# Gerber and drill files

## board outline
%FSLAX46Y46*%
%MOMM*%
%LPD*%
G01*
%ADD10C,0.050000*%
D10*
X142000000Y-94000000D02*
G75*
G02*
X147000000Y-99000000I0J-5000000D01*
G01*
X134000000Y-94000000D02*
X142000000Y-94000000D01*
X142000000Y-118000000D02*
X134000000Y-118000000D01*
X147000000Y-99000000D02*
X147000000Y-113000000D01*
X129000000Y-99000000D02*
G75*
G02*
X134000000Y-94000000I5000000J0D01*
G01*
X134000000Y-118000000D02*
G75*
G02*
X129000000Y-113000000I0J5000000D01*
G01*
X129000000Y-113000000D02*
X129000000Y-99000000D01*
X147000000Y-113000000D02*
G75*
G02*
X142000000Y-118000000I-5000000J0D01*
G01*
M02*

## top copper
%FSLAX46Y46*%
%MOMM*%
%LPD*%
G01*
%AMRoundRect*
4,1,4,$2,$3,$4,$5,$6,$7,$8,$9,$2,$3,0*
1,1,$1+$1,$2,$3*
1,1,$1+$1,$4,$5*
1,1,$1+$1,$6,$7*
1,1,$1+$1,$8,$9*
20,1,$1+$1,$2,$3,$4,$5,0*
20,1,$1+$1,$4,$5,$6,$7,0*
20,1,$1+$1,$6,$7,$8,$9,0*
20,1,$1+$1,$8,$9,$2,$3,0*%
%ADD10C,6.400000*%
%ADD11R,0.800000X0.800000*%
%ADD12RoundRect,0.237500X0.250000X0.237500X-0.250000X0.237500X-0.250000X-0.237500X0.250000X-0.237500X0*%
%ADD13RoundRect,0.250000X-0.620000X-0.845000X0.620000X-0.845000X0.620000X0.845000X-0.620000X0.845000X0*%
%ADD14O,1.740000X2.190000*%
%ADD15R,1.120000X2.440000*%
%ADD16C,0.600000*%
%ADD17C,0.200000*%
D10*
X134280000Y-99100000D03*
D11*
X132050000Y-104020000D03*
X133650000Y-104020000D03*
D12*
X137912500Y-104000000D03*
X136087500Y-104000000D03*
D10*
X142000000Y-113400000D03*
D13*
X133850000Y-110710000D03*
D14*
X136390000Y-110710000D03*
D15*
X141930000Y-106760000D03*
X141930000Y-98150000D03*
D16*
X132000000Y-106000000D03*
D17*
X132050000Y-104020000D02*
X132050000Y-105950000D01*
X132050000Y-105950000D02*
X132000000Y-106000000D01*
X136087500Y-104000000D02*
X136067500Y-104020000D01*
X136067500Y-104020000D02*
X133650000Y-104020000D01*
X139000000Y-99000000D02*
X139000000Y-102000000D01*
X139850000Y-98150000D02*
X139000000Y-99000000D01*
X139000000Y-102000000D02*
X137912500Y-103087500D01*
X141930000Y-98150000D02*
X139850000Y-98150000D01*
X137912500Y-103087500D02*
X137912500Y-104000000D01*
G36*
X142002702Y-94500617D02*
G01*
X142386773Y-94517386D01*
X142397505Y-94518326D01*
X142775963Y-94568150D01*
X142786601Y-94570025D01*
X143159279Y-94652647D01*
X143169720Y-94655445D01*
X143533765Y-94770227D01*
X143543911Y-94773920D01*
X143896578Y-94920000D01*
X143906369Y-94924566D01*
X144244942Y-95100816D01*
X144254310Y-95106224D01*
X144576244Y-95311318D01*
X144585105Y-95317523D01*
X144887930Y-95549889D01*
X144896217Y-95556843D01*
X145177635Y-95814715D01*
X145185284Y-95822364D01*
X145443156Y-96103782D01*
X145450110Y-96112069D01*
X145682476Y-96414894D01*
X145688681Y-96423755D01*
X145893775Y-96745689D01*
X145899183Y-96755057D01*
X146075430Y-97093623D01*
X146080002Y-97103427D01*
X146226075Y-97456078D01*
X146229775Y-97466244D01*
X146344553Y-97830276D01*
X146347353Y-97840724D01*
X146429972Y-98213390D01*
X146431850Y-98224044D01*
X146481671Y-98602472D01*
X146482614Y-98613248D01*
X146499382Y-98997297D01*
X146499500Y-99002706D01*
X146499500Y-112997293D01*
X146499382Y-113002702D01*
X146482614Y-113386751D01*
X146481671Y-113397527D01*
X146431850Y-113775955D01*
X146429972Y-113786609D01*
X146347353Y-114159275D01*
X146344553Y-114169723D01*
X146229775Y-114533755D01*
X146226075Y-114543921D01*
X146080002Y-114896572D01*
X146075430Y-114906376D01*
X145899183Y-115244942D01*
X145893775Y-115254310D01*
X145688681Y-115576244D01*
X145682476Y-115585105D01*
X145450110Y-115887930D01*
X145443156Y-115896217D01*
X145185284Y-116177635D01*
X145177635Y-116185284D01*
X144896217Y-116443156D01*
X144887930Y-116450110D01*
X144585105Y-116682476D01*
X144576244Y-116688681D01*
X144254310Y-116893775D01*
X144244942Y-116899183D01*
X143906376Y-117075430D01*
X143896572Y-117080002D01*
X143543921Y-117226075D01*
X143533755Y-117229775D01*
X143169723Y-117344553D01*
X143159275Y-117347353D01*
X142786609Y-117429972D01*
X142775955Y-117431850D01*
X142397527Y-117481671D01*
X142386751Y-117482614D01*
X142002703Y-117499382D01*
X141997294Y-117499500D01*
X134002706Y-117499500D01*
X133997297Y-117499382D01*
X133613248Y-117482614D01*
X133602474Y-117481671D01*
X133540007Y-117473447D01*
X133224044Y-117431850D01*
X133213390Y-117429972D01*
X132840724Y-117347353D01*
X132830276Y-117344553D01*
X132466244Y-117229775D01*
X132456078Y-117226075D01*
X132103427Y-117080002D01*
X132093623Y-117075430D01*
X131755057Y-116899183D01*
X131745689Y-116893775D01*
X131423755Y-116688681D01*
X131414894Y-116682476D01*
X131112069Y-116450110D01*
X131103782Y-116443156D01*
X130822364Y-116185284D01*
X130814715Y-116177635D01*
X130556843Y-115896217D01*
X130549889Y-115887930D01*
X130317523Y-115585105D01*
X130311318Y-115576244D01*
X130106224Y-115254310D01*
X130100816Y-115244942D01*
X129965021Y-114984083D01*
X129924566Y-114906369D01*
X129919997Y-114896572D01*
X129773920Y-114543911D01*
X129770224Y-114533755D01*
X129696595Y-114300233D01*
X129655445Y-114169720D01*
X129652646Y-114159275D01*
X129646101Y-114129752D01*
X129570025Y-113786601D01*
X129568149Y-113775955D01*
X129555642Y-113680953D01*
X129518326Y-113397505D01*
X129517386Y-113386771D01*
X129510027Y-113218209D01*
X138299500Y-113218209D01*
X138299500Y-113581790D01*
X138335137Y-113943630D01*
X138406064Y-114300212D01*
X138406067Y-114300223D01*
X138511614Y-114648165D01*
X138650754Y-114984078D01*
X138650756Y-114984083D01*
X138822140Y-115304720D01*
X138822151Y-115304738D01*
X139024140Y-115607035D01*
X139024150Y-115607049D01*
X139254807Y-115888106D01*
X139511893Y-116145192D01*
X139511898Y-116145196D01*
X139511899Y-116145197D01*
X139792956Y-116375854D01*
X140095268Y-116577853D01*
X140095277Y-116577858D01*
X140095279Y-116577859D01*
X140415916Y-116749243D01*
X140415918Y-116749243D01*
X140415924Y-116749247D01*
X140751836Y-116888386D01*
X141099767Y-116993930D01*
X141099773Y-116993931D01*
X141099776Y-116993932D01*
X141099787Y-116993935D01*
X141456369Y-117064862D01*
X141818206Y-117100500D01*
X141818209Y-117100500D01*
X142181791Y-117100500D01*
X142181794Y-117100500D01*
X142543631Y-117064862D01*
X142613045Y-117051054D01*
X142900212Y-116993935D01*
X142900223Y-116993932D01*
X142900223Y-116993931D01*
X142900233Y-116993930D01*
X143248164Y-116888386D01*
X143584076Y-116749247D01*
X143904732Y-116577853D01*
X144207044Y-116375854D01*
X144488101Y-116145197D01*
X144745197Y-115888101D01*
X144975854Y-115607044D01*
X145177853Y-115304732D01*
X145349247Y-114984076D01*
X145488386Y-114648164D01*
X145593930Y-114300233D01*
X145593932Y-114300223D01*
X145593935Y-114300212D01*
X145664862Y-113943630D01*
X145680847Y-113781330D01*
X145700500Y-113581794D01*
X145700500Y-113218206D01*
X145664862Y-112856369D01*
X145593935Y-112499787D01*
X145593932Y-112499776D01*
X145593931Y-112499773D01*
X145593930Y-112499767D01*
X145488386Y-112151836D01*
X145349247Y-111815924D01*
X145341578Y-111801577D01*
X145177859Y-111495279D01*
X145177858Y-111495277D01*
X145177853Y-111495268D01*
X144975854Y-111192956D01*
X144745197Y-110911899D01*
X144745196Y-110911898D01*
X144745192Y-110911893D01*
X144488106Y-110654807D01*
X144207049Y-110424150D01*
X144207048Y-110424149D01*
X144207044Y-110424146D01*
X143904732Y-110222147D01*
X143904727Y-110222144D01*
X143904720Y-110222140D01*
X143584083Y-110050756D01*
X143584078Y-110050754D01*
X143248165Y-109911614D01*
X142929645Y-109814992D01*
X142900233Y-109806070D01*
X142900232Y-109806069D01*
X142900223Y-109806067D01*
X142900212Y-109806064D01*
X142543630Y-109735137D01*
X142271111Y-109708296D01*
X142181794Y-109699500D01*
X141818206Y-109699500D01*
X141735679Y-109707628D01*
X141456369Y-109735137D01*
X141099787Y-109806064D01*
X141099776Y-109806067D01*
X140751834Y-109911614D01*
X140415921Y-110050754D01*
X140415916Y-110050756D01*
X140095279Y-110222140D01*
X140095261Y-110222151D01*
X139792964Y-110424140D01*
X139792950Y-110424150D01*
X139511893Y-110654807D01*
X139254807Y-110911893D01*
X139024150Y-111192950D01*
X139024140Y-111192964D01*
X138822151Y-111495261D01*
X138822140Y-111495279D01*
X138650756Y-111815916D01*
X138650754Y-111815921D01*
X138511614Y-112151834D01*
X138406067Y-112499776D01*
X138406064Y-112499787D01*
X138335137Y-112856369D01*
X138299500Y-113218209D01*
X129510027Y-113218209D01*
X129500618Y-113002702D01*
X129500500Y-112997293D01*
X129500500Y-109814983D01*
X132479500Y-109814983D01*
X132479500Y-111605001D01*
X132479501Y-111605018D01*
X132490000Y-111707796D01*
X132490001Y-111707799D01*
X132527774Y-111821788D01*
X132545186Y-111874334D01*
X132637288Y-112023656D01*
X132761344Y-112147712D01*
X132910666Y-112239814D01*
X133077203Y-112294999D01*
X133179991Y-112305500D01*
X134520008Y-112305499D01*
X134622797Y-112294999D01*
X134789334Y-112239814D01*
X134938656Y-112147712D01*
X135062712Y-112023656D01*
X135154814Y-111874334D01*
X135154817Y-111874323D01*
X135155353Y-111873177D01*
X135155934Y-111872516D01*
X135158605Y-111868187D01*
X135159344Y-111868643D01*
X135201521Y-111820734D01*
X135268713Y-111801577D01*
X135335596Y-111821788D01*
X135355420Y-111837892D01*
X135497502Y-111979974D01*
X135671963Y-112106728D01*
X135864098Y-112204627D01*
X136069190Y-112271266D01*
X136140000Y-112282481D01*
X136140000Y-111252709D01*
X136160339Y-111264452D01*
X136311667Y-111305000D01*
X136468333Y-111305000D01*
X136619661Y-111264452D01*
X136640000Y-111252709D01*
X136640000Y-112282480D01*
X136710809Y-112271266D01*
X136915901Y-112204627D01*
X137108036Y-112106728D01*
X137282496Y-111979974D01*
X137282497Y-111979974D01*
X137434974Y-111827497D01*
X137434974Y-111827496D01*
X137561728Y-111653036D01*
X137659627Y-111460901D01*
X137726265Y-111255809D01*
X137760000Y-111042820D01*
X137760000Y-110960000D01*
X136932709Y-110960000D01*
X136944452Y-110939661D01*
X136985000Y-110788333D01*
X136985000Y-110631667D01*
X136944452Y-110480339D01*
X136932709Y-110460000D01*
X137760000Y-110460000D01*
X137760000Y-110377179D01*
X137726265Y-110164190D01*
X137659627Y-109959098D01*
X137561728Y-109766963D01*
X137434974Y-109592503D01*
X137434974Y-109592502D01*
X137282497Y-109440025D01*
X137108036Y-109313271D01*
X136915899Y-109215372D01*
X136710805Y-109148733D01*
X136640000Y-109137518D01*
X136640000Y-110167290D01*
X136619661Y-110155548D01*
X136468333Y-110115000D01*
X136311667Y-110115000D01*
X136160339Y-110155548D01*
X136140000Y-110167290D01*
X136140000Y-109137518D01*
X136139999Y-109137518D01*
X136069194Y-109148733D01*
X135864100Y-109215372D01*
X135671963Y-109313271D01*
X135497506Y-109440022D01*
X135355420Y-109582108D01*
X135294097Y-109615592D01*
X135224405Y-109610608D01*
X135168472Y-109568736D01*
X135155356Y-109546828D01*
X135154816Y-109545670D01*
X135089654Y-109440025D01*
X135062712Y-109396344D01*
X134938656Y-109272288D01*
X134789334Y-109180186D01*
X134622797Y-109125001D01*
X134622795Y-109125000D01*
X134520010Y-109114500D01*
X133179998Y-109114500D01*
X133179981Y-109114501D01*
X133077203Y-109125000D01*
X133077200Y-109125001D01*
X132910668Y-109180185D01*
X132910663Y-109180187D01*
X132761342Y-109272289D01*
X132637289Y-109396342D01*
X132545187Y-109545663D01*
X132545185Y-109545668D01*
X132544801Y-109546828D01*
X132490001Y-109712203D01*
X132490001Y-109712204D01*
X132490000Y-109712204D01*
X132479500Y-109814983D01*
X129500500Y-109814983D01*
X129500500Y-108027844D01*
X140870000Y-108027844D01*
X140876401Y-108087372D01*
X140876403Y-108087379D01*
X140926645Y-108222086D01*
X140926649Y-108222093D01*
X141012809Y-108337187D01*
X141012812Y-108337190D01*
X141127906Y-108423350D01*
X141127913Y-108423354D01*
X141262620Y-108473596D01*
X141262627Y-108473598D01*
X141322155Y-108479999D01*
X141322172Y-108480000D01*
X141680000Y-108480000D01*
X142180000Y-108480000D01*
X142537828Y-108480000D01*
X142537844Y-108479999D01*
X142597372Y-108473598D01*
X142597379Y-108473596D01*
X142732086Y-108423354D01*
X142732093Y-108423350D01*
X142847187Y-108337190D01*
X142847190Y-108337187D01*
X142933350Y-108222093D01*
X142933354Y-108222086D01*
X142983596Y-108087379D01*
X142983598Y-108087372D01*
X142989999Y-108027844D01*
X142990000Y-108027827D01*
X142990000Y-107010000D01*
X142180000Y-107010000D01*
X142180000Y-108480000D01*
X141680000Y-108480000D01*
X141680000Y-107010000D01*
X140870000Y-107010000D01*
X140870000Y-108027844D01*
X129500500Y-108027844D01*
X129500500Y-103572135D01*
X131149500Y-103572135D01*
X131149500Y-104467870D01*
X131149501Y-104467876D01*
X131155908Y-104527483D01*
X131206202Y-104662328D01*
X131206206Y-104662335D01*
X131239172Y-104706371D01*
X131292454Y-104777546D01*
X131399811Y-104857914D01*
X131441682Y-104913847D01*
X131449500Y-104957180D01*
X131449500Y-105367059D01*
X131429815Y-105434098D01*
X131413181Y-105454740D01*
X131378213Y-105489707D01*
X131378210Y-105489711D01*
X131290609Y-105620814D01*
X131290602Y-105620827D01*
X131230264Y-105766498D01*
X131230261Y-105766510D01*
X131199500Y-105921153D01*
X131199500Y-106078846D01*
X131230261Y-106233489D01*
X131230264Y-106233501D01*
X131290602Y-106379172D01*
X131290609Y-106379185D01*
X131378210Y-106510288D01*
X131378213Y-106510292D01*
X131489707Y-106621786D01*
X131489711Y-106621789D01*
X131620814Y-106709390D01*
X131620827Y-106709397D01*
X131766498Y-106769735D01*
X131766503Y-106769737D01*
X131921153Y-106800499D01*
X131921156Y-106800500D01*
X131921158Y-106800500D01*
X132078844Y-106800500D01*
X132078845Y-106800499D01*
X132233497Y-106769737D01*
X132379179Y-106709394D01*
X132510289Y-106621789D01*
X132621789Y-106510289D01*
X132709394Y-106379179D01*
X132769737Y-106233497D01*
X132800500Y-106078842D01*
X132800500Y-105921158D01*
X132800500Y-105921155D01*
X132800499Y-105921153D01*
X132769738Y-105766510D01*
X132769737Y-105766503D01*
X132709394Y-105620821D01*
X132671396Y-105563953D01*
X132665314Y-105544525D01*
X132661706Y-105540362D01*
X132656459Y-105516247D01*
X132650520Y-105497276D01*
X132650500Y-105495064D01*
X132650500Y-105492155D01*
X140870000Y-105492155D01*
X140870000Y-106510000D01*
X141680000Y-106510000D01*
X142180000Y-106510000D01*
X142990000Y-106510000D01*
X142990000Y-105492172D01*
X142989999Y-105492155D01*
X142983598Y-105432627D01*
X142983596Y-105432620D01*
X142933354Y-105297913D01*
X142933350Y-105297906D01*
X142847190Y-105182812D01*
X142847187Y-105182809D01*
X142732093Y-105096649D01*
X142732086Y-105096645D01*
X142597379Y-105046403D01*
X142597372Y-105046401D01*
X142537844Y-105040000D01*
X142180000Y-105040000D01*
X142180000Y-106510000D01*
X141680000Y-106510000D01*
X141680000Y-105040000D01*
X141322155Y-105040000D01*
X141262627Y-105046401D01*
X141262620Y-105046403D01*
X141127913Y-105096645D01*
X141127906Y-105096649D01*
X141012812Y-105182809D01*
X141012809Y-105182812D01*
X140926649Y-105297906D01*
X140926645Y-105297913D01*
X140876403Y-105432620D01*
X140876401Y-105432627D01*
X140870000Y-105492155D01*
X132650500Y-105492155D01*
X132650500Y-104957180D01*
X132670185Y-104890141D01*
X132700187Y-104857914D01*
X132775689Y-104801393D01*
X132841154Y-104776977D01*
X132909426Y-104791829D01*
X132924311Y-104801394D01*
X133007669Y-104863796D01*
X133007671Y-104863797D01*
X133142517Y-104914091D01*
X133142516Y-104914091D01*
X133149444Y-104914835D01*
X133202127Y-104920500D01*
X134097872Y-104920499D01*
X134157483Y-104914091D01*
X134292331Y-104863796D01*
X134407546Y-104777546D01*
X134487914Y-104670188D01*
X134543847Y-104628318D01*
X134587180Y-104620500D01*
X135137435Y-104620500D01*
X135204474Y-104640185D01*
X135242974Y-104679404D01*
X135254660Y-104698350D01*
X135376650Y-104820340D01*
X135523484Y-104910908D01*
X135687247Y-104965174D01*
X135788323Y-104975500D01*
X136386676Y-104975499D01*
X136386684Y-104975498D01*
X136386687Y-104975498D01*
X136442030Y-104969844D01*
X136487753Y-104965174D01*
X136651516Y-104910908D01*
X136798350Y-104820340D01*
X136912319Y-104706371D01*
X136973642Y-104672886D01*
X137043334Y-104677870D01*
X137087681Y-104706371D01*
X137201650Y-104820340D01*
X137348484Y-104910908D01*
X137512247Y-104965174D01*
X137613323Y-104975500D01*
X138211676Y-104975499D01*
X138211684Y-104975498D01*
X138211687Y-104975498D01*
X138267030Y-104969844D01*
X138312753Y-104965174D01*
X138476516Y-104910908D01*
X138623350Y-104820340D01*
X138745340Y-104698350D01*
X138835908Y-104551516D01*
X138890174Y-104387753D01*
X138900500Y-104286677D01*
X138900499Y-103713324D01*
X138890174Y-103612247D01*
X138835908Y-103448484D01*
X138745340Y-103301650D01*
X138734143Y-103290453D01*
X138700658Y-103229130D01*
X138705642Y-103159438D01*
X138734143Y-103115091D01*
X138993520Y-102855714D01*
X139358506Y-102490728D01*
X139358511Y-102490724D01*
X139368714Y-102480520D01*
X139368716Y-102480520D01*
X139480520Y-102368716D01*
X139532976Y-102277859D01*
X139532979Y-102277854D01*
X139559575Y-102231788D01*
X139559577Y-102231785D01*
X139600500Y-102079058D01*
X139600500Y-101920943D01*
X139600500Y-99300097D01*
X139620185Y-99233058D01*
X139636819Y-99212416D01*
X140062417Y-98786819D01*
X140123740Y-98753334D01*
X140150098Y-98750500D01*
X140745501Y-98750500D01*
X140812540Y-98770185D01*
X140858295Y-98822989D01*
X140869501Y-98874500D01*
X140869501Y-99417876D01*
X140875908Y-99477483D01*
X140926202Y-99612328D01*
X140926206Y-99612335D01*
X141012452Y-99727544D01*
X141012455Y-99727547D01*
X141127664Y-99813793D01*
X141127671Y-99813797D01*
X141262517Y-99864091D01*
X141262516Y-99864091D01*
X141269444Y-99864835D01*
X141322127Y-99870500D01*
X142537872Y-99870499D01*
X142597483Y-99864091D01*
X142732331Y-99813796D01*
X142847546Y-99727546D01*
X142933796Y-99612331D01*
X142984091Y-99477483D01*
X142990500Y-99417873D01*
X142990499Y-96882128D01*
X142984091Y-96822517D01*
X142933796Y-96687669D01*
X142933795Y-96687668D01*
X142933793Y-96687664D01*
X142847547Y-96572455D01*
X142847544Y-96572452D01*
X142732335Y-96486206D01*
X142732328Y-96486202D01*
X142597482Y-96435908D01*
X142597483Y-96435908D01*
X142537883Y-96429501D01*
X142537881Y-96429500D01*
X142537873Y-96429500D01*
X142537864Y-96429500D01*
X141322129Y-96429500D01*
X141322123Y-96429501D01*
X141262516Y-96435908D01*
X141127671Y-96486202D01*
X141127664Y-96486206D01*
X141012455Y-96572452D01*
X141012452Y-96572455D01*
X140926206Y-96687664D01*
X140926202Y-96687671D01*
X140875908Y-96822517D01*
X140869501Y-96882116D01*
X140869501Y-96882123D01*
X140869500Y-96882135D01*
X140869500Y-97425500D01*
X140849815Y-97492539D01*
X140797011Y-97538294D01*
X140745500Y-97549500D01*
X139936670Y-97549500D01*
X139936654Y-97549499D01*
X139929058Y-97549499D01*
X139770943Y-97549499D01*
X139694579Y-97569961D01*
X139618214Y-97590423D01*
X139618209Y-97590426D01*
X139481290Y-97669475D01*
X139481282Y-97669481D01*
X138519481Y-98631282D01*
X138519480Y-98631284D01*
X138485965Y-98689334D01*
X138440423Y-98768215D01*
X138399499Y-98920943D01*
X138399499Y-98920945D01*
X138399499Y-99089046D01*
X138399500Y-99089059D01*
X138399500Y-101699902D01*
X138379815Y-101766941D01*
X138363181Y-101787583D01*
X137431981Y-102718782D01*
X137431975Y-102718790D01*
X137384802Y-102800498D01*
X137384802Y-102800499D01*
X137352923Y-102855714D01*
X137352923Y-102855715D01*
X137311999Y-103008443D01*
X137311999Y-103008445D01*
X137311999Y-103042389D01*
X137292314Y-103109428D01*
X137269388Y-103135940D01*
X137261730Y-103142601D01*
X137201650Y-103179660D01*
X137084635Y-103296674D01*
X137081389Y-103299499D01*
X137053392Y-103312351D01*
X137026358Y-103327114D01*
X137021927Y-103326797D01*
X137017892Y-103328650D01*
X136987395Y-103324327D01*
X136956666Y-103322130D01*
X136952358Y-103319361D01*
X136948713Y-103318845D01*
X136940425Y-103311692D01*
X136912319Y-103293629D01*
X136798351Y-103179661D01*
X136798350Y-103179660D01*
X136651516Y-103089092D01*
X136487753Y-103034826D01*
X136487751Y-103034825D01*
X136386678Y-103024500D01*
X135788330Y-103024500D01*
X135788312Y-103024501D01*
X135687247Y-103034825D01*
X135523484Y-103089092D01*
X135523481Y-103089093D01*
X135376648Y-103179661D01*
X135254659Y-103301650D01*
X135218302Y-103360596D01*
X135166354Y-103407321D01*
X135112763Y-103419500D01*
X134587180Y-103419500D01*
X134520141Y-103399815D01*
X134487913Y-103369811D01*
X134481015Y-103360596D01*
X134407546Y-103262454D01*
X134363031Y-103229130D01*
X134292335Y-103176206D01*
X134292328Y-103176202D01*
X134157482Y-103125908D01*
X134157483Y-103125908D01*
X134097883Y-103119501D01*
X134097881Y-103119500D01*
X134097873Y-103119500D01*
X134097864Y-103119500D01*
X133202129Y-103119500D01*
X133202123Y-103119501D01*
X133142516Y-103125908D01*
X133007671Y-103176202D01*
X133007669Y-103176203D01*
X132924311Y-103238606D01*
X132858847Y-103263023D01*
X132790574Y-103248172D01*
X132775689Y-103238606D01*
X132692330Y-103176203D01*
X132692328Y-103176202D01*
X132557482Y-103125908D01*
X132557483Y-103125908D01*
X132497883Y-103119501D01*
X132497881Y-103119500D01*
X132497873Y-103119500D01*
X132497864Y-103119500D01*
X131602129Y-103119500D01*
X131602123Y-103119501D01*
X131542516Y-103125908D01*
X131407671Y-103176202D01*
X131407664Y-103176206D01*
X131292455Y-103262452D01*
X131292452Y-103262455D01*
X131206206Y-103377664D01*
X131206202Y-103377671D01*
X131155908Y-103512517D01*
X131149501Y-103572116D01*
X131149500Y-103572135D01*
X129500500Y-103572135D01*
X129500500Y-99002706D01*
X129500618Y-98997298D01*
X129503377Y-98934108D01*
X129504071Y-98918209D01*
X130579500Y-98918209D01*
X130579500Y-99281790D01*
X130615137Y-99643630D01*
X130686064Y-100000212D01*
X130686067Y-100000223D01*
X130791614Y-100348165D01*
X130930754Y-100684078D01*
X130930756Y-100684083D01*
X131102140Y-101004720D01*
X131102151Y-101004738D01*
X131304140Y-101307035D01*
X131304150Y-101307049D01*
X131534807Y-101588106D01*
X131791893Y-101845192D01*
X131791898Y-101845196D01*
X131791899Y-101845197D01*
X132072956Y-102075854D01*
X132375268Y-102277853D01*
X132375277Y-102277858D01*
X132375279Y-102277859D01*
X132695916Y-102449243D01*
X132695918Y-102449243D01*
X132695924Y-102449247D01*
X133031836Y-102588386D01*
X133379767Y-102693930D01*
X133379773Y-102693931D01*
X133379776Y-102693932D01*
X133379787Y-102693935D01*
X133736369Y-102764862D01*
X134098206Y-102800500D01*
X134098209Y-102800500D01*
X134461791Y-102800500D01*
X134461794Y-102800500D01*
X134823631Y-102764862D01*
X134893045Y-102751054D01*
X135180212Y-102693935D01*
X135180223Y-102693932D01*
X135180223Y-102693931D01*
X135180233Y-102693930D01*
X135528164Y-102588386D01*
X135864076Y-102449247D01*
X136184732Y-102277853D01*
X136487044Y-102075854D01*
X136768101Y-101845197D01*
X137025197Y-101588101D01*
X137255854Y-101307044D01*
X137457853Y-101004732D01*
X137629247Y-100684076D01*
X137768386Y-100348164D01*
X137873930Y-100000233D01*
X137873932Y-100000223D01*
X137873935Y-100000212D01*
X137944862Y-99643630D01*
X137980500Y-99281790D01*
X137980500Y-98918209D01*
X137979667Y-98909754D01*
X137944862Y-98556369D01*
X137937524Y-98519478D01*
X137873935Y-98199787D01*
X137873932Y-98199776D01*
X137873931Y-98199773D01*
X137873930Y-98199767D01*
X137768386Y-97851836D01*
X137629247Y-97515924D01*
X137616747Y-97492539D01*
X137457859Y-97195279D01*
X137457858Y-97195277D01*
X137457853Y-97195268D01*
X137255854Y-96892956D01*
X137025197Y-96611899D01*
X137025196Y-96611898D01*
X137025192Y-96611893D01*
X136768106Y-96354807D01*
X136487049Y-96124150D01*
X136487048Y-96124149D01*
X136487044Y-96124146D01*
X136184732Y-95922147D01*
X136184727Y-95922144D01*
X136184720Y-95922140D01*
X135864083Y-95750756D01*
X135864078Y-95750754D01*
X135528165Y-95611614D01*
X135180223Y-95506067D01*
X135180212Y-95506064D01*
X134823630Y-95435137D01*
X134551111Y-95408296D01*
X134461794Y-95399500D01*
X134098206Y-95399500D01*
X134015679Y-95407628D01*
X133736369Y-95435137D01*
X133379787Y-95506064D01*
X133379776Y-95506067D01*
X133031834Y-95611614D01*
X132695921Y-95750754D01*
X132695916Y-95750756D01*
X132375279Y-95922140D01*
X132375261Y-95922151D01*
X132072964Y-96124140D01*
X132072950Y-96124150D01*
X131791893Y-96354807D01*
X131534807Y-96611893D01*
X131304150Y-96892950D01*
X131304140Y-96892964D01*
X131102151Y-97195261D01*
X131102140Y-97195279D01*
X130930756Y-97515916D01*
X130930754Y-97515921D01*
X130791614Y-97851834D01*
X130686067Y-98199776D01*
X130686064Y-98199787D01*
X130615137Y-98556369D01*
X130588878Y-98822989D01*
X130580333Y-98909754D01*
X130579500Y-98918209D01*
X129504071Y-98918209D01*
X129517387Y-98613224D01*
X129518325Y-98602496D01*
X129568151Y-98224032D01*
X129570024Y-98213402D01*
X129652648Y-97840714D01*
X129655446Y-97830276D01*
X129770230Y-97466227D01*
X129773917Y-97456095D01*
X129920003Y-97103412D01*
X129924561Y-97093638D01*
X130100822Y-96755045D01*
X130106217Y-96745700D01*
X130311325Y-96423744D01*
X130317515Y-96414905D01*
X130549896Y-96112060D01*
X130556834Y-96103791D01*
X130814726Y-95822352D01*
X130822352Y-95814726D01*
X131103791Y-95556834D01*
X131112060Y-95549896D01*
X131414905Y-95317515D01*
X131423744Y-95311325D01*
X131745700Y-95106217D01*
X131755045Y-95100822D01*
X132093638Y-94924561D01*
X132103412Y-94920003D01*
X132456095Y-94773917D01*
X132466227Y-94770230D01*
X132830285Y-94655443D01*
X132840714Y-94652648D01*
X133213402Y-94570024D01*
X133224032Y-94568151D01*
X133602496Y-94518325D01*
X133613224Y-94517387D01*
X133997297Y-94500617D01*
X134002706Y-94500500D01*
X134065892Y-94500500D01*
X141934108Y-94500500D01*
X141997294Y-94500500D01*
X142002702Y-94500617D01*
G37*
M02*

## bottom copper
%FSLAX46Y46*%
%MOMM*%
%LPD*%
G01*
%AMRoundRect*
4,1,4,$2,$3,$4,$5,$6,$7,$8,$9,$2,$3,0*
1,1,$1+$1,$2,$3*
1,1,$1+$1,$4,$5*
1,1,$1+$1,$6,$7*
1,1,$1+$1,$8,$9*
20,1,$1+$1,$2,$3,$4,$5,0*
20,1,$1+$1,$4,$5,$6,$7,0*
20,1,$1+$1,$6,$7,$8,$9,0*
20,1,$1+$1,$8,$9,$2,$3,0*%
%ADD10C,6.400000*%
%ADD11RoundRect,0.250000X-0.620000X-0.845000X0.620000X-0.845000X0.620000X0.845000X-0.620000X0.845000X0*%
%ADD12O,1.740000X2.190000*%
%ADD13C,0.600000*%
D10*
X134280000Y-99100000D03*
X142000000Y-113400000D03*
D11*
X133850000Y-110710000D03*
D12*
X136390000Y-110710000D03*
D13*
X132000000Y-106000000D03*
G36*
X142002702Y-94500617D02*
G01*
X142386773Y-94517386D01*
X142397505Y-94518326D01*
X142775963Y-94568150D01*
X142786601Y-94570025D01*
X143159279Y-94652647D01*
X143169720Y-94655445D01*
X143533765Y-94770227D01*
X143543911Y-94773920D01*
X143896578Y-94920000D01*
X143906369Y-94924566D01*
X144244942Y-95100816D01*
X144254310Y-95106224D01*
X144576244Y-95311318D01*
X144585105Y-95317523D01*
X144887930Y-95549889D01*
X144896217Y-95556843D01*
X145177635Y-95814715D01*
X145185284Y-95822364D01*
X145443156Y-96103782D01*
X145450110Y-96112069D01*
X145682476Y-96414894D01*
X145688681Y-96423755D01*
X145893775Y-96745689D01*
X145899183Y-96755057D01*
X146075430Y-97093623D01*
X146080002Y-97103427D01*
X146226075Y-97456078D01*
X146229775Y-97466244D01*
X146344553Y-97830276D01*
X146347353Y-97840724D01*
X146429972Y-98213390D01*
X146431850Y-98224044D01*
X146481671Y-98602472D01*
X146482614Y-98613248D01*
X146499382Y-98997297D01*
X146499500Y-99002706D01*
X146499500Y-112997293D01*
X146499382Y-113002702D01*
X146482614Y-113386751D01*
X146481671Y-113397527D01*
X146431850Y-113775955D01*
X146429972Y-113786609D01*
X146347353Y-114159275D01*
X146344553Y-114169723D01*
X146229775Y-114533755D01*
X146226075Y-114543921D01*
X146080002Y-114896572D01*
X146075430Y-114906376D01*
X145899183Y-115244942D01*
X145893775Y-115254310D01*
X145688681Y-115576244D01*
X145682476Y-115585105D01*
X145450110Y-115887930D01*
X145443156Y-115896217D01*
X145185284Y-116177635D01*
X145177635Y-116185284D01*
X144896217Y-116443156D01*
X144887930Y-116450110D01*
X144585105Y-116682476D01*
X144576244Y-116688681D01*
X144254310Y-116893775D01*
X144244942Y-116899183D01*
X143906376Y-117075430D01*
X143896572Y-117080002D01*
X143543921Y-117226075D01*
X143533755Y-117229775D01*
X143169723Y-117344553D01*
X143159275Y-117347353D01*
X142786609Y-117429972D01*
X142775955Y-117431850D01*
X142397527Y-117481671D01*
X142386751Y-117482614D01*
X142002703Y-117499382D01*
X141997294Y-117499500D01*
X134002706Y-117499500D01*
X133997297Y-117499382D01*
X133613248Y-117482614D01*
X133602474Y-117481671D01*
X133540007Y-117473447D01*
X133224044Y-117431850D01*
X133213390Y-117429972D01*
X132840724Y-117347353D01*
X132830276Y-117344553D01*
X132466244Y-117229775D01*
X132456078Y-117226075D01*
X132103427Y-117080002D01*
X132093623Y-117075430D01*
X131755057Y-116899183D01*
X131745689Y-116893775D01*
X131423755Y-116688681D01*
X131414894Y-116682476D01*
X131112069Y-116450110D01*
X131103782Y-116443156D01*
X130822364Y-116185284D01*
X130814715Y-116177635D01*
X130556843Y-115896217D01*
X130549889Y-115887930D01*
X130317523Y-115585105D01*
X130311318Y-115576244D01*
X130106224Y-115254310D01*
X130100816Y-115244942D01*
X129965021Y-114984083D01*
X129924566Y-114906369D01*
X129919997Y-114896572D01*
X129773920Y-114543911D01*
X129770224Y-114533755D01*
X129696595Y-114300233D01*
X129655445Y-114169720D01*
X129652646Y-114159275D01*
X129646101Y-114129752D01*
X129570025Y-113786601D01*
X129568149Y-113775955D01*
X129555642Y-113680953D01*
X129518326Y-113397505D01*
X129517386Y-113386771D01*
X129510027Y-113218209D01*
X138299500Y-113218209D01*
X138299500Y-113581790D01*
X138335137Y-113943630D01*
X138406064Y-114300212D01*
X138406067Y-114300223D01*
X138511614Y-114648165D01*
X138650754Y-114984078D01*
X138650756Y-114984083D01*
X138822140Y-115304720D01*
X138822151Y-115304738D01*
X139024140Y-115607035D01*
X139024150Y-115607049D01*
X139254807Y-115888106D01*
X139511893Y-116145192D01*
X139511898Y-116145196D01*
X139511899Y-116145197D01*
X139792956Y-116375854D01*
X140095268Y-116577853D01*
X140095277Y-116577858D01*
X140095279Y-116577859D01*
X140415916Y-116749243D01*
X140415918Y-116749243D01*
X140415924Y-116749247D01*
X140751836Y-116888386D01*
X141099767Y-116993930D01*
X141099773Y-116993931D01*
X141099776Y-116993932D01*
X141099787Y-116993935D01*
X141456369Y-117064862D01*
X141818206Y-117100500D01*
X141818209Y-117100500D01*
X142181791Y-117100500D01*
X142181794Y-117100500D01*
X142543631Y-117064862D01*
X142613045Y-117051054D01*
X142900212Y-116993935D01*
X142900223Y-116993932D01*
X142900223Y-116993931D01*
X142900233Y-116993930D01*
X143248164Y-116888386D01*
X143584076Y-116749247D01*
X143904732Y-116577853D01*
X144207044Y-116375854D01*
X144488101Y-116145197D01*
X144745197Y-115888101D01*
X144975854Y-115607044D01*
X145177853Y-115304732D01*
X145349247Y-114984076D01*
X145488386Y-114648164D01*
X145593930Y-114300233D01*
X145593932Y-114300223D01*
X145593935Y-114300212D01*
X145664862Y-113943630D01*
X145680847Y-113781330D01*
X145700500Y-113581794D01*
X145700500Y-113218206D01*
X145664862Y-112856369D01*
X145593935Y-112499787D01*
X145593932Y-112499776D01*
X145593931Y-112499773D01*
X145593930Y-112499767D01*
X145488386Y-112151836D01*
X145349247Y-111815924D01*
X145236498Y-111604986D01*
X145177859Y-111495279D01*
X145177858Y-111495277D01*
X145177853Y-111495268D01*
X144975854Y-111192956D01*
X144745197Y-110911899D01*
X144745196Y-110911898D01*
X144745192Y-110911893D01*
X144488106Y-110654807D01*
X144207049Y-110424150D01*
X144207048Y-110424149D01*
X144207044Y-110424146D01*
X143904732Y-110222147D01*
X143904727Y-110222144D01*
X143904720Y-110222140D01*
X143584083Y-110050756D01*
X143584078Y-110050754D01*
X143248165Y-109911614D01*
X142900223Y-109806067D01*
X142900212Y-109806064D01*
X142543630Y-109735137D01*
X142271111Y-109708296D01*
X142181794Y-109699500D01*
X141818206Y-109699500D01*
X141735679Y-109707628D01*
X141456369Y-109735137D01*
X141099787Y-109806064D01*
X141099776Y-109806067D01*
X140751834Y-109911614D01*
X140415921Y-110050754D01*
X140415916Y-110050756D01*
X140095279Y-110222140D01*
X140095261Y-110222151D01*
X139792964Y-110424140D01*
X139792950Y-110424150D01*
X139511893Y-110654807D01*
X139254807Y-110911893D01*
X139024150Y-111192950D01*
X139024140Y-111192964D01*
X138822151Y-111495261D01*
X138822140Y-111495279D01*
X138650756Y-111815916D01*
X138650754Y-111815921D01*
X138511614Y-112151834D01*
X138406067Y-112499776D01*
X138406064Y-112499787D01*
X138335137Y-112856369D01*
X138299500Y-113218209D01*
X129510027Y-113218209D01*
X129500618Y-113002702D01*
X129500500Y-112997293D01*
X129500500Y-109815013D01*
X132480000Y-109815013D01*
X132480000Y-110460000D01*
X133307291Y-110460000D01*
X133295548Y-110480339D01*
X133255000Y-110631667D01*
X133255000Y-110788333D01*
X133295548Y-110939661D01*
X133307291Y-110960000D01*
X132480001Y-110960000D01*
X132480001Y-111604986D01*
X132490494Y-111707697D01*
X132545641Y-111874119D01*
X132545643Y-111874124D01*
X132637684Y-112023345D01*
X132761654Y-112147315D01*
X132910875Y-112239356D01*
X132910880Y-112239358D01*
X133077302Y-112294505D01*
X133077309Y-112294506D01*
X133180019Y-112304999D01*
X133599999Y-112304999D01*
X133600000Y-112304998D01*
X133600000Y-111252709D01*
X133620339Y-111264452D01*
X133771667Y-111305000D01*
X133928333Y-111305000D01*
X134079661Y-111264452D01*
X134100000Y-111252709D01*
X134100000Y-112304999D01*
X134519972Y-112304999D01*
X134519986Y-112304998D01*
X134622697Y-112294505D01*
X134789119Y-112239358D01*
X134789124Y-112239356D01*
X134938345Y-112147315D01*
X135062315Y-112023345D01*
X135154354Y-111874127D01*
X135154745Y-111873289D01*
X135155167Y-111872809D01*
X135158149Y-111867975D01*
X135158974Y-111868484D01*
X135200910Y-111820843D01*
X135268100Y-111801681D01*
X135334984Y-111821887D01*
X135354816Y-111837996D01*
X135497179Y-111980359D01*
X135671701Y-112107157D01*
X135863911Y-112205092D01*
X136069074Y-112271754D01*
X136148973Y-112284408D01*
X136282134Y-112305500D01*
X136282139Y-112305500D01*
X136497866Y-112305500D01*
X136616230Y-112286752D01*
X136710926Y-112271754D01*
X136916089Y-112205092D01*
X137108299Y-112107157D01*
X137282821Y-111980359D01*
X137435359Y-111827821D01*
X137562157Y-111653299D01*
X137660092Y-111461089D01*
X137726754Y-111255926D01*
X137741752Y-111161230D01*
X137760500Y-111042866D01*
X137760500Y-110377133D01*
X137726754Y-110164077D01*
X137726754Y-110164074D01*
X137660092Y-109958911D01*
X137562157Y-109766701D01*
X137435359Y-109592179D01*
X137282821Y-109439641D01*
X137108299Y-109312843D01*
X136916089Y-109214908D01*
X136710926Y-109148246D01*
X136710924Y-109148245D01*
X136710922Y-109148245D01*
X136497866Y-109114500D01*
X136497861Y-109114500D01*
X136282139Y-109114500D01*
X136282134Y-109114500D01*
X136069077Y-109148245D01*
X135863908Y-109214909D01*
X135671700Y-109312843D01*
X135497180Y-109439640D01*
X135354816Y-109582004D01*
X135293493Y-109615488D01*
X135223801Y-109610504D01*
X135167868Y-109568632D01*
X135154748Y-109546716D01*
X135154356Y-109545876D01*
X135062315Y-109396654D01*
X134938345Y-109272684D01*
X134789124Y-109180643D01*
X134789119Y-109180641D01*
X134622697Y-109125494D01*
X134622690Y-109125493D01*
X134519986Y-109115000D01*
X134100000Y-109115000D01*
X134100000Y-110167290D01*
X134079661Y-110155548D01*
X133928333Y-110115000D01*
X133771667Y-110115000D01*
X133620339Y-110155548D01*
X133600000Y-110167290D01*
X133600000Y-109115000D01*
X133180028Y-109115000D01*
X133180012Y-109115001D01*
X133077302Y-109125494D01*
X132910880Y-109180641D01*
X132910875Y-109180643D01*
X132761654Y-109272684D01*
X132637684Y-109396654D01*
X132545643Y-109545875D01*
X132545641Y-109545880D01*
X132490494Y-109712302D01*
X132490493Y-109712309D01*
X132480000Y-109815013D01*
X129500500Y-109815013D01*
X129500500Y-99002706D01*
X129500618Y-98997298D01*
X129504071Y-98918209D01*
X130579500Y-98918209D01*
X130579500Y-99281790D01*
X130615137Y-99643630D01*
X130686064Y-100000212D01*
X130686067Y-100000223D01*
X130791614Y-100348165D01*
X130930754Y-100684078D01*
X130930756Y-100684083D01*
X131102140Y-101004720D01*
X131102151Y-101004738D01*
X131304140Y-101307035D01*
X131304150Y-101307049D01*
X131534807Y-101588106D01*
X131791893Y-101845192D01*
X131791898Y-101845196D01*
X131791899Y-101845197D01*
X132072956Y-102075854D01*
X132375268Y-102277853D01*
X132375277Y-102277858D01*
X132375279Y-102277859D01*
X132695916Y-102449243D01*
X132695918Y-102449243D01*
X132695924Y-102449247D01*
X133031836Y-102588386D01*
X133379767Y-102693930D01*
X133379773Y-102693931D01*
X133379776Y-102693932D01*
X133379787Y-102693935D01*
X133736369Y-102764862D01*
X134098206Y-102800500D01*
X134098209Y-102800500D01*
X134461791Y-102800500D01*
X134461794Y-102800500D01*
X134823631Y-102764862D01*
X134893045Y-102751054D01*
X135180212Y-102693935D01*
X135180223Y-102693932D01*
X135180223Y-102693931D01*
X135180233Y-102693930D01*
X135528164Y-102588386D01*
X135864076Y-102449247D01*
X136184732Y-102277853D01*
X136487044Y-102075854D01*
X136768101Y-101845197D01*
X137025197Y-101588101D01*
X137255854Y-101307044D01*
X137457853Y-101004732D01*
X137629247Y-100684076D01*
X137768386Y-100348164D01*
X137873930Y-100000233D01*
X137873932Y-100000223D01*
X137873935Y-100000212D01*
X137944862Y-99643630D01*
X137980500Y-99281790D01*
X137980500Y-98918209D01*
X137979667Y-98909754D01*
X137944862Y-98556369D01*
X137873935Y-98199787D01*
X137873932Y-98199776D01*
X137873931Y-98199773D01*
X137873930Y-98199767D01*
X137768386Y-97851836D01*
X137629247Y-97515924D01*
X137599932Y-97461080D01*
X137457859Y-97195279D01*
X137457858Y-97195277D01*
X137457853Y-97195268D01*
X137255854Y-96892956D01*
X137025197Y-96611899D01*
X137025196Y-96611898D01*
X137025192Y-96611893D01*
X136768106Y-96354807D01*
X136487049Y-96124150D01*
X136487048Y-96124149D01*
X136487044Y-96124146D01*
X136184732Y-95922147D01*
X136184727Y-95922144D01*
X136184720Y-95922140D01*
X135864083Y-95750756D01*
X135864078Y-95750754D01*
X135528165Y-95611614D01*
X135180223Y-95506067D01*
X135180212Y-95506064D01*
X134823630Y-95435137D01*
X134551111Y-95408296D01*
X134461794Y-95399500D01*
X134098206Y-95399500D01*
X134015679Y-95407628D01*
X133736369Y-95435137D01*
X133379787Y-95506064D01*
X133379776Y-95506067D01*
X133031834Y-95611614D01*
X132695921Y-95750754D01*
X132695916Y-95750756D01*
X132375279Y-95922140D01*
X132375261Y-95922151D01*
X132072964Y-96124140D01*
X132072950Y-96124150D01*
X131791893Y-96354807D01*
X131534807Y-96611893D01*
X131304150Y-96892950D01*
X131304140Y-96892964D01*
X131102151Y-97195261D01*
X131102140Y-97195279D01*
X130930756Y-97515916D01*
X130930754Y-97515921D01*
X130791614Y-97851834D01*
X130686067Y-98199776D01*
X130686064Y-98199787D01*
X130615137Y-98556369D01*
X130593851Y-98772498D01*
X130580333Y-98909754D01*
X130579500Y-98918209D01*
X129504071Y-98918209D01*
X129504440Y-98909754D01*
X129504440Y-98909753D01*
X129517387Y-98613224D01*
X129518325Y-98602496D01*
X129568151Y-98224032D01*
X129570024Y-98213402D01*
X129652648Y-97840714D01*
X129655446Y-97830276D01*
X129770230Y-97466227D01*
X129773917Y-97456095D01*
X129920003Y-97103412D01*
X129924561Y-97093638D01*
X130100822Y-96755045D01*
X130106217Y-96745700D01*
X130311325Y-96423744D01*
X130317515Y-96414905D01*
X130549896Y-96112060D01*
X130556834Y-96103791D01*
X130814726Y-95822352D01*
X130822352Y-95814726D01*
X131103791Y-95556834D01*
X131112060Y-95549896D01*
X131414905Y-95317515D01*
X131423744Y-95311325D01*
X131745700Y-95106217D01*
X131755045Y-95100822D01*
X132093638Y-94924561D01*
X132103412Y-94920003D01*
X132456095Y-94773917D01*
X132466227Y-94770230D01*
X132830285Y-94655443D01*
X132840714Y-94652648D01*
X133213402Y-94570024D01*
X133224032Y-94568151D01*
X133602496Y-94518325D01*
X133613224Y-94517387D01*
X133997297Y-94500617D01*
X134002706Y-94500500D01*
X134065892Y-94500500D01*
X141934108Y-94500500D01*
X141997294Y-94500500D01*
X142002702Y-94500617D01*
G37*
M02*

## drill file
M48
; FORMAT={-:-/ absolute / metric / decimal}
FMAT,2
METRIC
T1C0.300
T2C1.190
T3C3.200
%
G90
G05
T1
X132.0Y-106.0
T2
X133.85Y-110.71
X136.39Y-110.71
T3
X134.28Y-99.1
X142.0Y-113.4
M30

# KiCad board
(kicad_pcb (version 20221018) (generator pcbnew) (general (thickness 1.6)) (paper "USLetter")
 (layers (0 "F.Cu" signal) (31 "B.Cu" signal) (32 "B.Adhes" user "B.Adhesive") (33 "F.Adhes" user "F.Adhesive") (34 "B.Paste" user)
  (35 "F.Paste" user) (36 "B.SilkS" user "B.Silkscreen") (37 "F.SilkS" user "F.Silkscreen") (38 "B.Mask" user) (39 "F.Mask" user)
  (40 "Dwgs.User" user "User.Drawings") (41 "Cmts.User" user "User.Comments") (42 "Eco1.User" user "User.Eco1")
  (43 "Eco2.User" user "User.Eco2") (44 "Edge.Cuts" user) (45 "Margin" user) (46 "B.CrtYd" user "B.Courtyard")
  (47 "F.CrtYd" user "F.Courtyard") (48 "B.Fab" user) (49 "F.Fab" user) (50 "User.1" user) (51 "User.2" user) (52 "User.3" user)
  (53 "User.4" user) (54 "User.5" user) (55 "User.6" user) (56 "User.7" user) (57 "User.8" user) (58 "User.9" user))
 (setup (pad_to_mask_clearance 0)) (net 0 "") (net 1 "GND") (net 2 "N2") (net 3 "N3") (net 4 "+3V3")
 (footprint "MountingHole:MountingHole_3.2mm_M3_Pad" (layer "F.Cu") (at 134.28 99.1)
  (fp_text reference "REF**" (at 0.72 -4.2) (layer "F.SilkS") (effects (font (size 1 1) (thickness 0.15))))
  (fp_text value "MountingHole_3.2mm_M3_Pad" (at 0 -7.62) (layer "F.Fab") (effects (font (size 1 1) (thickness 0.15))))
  (pad "1" thru_hole circle (at 0 0) (size 6.4 6.4) (drill 3.2) (layers "*.Cu" "*.Mask")))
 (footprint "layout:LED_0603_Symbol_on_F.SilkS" (layer "F.Cu") (at 132.85 104.02)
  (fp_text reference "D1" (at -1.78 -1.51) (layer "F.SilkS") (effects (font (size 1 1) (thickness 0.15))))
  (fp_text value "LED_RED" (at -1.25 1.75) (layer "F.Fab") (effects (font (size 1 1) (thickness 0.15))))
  (pad "1" smd rect (at -0.8 0 180) (size 0.8 0.8) (layers "F.Cu" "F.Paste" "F.Mask") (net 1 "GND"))
  (pad "2" smd rect (at 0.8 0 180) (size 0.8 0.8) (layers "F.Cu" "F.Paste" "F.Mask") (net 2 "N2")))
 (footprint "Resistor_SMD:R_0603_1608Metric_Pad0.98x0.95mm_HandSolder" (layer "F.Cu") (at 137 104 180)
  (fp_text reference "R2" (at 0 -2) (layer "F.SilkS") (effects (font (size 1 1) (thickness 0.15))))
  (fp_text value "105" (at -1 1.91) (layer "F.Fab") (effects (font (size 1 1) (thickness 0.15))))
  (pad "1" smd roundrect (at -0.9125 0 180) (size 0.975 0.95) (layers "F.Cu" "F.Paste" "F.Mask") (roundrect_rratio 0.25) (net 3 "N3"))
  (pad "2" smd roundrect (at 0.9125 0 180) (size 0.975 0.95) (layers "F.Cu" "F.Paste" "F.Mask") (roundrect_rratio 0.25) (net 2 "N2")))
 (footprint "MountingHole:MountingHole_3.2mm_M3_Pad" (layer "F.Cu") (at 142 113.4)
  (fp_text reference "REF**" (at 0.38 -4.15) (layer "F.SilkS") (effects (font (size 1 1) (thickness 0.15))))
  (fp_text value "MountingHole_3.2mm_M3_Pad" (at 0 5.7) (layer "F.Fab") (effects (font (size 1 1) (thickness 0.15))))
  (pad "1" thru_hole circle (at 0 0) (size 6.4 6.4) (drill 3.2) (layers "*.Cu" "*.Mask")))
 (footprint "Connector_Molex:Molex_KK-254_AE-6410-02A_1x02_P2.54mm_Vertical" (layer "F.Cu") (at 133.85 110.71)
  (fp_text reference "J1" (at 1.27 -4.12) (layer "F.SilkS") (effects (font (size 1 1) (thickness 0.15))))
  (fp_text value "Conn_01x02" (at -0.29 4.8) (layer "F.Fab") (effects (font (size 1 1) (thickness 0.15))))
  (pad "1" thru_hole roundrect (at 0 0) (size 1.74 2.19) (drill 1.19) (layers "*.Cu" "*.Mask") (roundrect_rratio 0.143678) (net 1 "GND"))
  (pad "2" thru_hole oval (at 2.54 0) (size 1.74 2.19) (drill 1.19) (layers "*.Cu" "*.Mask") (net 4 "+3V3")))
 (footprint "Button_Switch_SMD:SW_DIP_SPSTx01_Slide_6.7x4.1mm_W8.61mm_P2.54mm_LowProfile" (layer "F.Cu") (at 141.93 102.455 90)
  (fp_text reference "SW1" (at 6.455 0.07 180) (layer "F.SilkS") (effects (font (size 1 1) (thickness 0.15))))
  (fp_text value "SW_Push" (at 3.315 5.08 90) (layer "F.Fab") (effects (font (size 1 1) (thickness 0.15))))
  (pad "1" smd rect (at -4.305 0 90) (size 2.44 1.12) (layers "F.Cu" "F.Paste" "F.Mask") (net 4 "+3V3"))
  (pad "2" smd rect (at 4.305 0 90) (size 2.44 1.12) (layers "F.Cu" "F.Paste" "F.Mask") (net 3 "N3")))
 (gr_arc (start 142 94) (mid 145.535534 95.464466) (end 147 99) (stroke (width 0.05) (type default)) (layer "Edge.Cuts"))
 (gr_line (start 134 94) (end 142 94) (stroke (width 0.05) (type default)) (layer "Edge.Cuts"))
 (gr_line (start 142 118) (end 134 118) (stroke (width 0.05) (type default)) (layer "Edge.Cuts"))
 (gr_line (start 147 99) (end 147 113) (stroke (width 0.05) (type default)) (layer "Edge.Cuts"))
 (gr_arc (start 129 99) (mid 130.464466 95.464466) (end 134 94) (stroke (width 0.05) (type default)) (layer "Edge.Cuts"))
 (gr_arc (start 134 118) (mid 130.464466 116.535534) (end 129 113) (stroke (width 0.05) (type default)) (layer "Edge.Cuts"))
 (gr_line (start 129 113) (end 129 99) (stroke (width 0.05) (type default)) (layer "Edge.Cuts"))
 (gr_arc (start 147 113) (mid 145.535534 116.535534) (end 142 118) (stroke (width 0.05) (type default)) (layer "Edge.Cuts"))
 (segment (start 132.05 104.02) (end 132.05 105.95) (width 0.2) (layer "F.Cu") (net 1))
 (segment (start 132.05 105.95) (end 132 106) (width 0.2) (layer "F.Cu") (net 1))
 (via (at 132 106) (size 0.6) (drill 0.3) (layers "F.Cu" "B.Cu") (free) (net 1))
 (segment (start 136.0875 104) (end 136.0675 104.02) (width 0.2) (layer "F.Cu") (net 2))
 (segment (start 136.0675 104.02) (end 133.65 104.02) (width 0.2) (layer "F.Cu") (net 2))
 (segment (start 139 99) (end 139 102) (width 0.2) (layer "F.Cu") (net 3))
 (segment (start 139.85 98.15) (end 139 99) (width 0.2) (layer "F.Cu") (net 3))
 (segment (start 139 102) (end 137.9125 103.0875) (width 0.2) (layer "F.Cu") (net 3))
 (segment (start 141.93 98.15) (end 139.85 98.15) (width 0.2) (layer "F.Cu") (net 3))
 (segment (start 137.9125 103.0875) (end 137.9125 104) (width 0.2) (layer "F.Cu") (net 3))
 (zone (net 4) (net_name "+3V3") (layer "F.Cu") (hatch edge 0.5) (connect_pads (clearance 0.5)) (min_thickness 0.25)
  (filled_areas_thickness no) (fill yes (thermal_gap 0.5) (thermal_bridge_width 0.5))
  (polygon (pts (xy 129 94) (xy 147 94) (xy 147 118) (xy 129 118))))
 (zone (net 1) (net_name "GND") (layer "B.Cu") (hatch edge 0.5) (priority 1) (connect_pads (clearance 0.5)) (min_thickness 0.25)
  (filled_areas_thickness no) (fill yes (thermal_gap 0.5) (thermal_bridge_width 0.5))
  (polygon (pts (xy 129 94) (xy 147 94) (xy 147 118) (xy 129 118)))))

